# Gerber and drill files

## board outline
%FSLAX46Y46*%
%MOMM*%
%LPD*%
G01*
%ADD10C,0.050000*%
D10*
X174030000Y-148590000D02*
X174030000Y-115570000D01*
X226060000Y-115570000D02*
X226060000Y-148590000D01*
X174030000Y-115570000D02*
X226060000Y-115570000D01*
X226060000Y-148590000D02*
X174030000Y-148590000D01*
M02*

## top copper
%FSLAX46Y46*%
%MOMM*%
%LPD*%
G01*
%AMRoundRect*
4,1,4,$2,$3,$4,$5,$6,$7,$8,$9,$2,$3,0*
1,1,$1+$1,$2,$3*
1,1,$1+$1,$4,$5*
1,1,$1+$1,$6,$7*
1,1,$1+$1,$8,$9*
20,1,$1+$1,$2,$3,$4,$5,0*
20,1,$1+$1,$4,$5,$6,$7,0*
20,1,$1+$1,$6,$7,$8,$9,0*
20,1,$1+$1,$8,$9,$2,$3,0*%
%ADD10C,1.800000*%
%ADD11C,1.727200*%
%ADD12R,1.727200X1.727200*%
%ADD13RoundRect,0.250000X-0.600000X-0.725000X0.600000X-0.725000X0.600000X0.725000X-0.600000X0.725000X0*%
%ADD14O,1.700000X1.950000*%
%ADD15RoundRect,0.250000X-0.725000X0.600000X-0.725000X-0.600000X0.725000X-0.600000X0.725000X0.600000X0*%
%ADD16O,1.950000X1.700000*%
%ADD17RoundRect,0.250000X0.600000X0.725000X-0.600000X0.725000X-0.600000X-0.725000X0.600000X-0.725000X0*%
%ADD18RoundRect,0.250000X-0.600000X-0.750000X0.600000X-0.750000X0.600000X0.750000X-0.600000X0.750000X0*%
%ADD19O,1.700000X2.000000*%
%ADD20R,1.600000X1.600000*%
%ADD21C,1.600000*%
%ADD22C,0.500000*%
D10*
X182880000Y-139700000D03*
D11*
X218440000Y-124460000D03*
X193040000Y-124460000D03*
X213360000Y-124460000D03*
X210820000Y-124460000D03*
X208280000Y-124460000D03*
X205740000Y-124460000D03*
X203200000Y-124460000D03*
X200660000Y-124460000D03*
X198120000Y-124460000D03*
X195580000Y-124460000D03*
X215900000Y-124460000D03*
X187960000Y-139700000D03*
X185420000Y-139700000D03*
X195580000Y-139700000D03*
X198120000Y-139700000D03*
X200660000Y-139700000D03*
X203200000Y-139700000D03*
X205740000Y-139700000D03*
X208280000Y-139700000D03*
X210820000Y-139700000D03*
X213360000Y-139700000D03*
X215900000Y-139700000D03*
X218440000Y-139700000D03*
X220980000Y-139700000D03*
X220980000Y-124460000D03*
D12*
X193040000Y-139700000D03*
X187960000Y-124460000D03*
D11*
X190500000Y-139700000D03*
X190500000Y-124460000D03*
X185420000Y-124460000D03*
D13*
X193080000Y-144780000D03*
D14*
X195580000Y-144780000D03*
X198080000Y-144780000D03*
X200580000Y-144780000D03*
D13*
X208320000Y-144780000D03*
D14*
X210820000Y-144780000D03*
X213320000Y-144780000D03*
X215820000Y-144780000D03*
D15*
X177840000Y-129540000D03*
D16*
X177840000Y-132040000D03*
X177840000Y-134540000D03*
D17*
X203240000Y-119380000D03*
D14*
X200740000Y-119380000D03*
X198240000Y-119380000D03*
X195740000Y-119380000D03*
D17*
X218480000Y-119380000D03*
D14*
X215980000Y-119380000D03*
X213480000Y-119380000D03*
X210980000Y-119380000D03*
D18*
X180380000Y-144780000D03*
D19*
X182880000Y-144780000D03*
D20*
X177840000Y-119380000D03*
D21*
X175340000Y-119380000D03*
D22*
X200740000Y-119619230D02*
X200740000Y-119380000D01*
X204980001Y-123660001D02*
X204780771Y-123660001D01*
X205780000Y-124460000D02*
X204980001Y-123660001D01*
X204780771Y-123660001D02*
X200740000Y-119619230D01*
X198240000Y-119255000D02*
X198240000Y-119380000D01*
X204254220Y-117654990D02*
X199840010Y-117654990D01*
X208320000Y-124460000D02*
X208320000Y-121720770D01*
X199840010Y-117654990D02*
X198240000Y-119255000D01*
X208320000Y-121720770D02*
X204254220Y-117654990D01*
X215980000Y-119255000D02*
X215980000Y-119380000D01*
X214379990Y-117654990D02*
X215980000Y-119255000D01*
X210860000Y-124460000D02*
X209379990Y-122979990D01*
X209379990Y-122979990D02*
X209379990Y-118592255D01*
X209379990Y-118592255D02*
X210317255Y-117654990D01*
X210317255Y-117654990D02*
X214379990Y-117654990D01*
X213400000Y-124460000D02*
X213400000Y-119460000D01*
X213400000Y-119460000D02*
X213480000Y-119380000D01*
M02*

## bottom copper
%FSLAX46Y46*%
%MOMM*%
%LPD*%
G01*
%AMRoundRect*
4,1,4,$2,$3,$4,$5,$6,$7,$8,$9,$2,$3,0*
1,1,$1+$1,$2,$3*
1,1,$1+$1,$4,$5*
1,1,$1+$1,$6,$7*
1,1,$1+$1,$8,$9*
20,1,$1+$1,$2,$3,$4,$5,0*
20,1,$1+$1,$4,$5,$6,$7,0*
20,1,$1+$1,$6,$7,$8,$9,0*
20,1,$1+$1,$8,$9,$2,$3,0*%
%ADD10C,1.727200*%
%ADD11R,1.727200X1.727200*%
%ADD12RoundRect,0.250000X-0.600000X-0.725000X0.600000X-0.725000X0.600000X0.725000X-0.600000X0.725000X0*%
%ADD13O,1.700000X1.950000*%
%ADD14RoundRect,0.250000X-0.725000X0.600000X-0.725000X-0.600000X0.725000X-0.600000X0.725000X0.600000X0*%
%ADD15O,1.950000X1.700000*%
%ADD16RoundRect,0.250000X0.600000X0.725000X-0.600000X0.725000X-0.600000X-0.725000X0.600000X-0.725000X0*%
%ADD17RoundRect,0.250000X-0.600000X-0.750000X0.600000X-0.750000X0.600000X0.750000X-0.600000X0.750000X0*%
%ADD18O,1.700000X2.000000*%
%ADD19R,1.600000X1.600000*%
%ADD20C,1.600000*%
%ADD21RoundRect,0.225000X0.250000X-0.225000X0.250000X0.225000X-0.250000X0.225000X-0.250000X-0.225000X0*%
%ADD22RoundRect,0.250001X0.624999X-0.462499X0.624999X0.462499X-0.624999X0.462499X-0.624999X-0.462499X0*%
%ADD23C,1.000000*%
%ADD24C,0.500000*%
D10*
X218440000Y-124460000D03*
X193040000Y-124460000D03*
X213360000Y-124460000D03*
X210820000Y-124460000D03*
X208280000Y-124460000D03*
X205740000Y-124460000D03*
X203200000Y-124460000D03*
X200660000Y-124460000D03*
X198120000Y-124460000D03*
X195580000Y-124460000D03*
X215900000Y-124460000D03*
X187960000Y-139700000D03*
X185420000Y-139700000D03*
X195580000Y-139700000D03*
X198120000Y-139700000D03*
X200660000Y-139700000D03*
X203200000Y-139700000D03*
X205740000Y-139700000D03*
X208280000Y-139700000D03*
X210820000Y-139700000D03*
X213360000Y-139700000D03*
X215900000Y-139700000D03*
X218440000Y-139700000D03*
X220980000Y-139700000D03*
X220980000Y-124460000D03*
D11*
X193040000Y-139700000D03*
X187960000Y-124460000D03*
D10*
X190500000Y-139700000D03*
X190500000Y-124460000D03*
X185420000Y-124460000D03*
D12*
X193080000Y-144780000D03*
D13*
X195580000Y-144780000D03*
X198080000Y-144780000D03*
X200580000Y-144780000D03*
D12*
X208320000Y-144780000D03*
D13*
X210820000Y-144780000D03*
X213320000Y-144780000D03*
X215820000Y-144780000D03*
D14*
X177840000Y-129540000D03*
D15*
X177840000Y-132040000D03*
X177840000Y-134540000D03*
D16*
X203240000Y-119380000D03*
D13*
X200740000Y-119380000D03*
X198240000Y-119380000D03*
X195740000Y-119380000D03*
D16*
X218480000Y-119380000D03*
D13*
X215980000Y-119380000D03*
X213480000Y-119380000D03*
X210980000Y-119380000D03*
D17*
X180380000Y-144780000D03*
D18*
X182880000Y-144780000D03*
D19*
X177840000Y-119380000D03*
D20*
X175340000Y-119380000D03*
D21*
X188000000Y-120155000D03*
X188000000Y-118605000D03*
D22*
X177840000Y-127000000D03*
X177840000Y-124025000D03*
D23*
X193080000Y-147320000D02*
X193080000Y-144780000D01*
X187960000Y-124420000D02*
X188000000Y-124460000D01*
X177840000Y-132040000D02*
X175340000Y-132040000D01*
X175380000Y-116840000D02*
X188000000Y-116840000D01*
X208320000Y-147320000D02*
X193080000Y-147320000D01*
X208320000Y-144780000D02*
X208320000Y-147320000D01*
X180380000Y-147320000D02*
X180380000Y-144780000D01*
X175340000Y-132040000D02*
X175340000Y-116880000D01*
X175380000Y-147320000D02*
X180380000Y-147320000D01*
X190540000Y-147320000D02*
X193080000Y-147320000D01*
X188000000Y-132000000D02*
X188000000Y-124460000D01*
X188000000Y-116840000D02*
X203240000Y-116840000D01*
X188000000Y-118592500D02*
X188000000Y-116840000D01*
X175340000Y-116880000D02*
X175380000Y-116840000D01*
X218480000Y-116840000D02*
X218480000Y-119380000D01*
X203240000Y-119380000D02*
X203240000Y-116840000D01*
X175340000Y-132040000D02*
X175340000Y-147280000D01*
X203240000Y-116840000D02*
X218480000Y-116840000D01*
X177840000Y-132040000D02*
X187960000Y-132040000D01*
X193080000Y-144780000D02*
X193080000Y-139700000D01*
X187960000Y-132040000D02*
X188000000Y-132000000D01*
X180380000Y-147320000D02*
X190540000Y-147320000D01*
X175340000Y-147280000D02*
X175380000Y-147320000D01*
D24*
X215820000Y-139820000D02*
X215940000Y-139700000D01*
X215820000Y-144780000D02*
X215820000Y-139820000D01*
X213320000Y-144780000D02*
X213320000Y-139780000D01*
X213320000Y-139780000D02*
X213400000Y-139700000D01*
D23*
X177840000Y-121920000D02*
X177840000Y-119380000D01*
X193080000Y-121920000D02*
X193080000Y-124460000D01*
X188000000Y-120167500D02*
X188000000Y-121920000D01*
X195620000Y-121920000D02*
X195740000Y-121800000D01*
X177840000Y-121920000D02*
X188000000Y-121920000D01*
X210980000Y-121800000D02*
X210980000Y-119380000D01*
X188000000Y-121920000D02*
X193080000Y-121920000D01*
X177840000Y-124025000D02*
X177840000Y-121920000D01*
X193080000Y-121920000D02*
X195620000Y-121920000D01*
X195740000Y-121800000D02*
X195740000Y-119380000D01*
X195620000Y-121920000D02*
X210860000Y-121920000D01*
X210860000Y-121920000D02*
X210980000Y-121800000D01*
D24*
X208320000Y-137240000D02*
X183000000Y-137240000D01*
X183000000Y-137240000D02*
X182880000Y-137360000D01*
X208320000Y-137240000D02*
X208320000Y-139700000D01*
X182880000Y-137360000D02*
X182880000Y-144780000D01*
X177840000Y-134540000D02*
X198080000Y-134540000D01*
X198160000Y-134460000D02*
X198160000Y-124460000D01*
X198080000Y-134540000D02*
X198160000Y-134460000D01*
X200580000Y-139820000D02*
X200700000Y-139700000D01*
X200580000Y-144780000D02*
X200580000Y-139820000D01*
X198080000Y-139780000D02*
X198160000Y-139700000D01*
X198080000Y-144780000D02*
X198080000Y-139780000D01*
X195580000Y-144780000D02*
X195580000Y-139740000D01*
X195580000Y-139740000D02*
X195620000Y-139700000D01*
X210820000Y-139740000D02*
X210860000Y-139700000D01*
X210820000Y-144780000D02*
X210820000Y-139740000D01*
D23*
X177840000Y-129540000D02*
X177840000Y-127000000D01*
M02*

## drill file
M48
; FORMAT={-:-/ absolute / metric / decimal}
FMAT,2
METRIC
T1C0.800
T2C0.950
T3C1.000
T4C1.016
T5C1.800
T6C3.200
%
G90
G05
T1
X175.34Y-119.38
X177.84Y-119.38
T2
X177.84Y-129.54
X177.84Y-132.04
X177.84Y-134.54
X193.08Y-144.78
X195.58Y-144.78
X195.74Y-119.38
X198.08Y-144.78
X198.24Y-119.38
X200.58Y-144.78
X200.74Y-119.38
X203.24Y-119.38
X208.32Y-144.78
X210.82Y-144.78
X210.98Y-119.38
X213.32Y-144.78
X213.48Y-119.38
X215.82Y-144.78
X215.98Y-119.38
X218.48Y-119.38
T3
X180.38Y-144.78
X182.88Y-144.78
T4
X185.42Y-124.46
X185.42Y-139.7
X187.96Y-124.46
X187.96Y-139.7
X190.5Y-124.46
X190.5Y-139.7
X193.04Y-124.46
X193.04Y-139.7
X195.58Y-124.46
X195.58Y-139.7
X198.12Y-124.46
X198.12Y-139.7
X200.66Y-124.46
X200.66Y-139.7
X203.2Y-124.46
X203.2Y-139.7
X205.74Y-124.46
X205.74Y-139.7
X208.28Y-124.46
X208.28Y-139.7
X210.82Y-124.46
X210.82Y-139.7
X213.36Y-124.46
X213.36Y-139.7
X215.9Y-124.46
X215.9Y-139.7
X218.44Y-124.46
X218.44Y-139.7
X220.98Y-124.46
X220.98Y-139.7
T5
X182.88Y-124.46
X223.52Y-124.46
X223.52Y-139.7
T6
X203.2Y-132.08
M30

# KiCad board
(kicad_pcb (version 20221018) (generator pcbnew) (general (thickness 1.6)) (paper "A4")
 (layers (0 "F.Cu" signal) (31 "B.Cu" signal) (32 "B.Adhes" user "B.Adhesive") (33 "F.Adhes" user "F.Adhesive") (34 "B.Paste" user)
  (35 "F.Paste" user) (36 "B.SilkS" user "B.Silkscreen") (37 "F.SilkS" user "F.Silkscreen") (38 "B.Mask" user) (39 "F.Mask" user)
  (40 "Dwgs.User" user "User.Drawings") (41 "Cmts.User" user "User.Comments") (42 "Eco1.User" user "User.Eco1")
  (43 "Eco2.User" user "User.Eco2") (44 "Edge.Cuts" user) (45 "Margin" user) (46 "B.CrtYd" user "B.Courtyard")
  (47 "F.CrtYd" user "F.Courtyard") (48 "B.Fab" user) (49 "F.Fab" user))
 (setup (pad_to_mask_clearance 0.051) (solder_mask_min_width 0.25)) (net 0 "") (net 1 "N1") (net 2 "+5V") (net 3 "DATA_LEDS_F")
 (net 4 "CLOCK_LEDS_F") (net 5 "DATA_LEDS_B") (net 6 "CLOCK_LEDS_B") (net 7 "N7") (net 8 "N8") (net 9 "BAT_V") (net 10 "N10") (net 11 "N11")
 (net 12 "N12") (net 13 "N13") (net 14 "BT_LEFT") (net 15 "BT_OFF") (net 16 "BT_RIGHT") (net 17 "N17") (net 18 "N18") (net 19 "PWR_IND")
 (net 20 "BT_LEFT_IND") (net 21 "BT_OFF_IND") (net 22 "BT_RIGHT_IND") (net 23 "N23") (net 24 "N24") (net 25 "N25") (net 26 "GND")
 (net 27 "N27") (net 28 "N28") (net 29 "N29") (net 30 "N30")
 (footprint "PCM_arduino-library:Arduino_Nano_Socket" (layer "F.Cu") (at 224.79 132.08 90)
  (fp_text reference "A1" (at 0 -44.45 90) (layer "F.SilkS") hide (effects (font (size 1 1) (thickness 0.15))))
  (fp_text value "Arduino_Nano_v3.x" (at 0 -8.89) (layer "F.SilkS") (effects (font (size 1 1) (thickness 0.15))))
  (pad "" connect circle (at -7.62 -41.91 90) (size 1.8 1.8) (layers "F.Cu" "F.Mask"))
  (pad "" np_thru_hole circle (at -7.62 -1.27 90) (size 1.8 1.8) (drill 1.8) (layers "F&B.Cu" "*.Mask"))
  (pad "" np_thru_hole circle (at 7.62 -41.91 90) (size 1.8 1.8) (drill 1.8) (layers "F&B.Cu" "*.Mask"))
  (pad "" np_thru_hole circle (at 7.62 -1.27 90) (size 1.8 1.8) (drill 1.8) (layers "F&B.Cu" "*.Mask"))
  (pad "3V3" thru_hole circle (at 7.62 -6.35 90) (size 1.7272 1.7272) (drill 1.016) (layers "*.Cu" "*.Mask") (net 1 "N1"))
  (pad "5V" thru_hole circle (at 7.62 -31.75 90) (size 1.7272 1.7272) (drill 1.016) (layers "*.Cu" "*.Mask") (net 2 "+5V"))
  (pad "A0" thru_hole circle (at 7.62 -11.43 90) (size 1.7272 1.7272) (drill 1.016) (layers "*.Cu" "*.Mask") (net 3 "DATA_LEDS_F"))
  (pad "A1" thru_hole circle (at 7.62 -13.97 90) (size 1.7272 1.7272) (drill 1.016) (layers "*.Cu" "*.Mask") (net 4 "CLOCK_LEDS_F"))
  (pad "A2" thru_hole circle (at 7.62 -16.51 90) (size 1.7272 1.7272) (drill 1.016) (layers "*.Cu" "*.Mask") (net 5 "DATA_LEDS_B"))
  (pad "A3" thru_hole circle (at 7.62 -19.05 90) (size 1.7272 1.7272) (drill 1.016) (layers "*.Cu" "*.Mask") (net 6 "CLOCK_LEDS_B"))
  (pad "A4" thru_hole circle (at 7.62 -21.59 90) (size 1.7272 1.7272) (drill 1.016) (layers "*.Cu" "*.Mask") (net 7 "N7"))
  (pad "A5" thru_hole circle (at 7.62 -24.13 90) (size 1.7272 1.7272) (drill 1.016) (layers "*.Cu" "*.Mask") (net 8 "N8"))
  (pad "A6" thru_hole circle (at 7.62 -26.67 90) (size 1.7272 1.7272) (drill 1.016) (layers "*.Cu" "*.Mask") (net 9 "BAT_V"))
  (pad "A7" thru_hole circle (at 7.62 -29.21 90) (size 1.7272 1.7272) (drill 1.016) (layers "*.Cu" "*.Mask") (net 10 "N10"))
  (pad "AREF" thru_hole circle (at 7.62 -8.89 90) (size 1.7272 1.7272) (drill 1.016) (layers "*.Cu" "*.Mask") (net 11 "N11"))
  (pad "D0" thru_hole circle (at -7.62 -36.83 90) (size 1.7272 1.7272) (drill 1.016) (layers "*.Cu" "*.Mask") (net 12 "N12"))
  (pad "D1" thru_hole circle (at -7.62 -39.37 90) (size 1.7272 1.7272) (drill 1.016) (layers "*.Cu" "*.Mask") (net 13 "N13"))
  (pad "D2" thru_hole circle (at -7.62 -29.21 90) (size 1.7272 1.7272) (drill 1.016) (layers "*.Cu" "*.Mask") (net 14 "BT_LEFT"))
  (pad "D3" thru_hole circle (at -7.62 -26.67 90) (size 1.7272 1.7272) (drill 1.016) (layers "*.Cu" "*.Mask") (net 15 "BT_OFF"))
  (pad "D4" thru_hole circle (at -7.62 -24.13 90) (size 1.7272 1.7272) (drill 1.016) (layers "*.Cu" "*.Mask") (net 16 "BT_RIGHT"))
  (pad "D5" thru_hole circle (at -7.62 -21.59 90) (size 1.7272 1.7272) (drill 1.016) (layers "*.Cu" "*.Mask") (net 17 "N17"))
  (pad "D6" thru_hole circle (at -7.62 -19.05 90) (size 1.7272 1.7272) (drill 1.016) (layers "*.Cu" "*.Mask") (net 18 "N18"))
  (pad "D7" thru_hole circle (at -7.62 -16.51 90) (size 1.7272 1.7272) (drill 1.016) (layers "*.Cu" "*.Mask") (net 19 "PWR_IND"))
  (pad "D8" thru_hole circle (at -7.62 -13.97 90) (size 1.7272 1.7272) (drill 1.016) (layers "*.Cu" "*.Mask") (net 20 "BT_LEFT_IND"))
  (pad "D9" thru_hole circle (at -7.62 -11.43 90) (size 1.7272 1.7272) (drill 1.016) (layers "*.Cu" "*.Mask") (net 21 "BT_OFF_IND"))
  (pad "D10" thru_hole circle (at -7.62 -8.89 90) (size 1.7272 1.7272) (drill 1.016) (layers "*.Cu" "*.Mask") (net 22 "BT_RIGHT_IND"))
  (pad "D11" thru_hole circle (at -7.62 -6.35 90) (size 1.7272 1.7272) (drill 1.016) (layers "*.Cu" "*.Mask") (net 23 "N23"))
  (pad "D12" thru_hole circle (at -7.62 -3.81 90) (size 1.7272 1.7272) (drill 1.016) (layers "*.Cu" "*.Mask") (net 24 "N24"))
  (pad "D13" thru_hole circle (at 7.62 -3.81 90) (size 1.7272 1.7272) (drill 1.016) (layers "*.Cu" "*.Mask") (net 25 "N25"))
  (pad "GND1" thru_hole rect (at -7.62 -31.75 90) (size 1.7272 1.7272) (drill 1.016) (layers "*.Cu" "*.Mask") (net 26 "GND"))
  (pad "GND2" thru_hole rect (at 7.62 -36.83 90) (size 1.7272 1.7272) (drill 1.016) (layers "*.Cu" "*.Mask") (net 26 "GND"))
  (pad "RST1" thru_hole circle (at -7.62 -34.29 90) (size 1.7272 1.7272) (drill 1.016) (layers "*.Cu" "*.Mask") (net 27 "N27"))
  (pad "RST2" thru_hole circle (at 7.62 -34.29 90) (size 1.7272 1.7272) (drill 1.016) (layers "*.Cu" "*.Mask") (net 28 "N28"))
  (pad "VIN" thru_hole circle (at 7.62 -39.37 90) (size 1.7272 1.7272) (drill 1.016) (layers "*.Cu" "*.Mask") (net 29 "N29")))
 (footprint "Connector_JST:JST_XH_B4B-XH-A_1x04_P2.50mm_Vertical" (layer "F.Cu") (at 193.08 144.78)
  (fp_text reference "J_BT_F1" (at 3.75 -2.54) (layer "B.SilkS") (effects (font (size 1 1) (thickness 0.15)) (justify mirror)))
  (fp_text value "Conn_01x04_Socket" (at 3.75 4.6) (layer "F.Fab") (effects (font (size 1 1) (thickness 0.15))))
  (pad "1" thru_hole roundrect (at 0 0) (size 1.7 1.95) (drill 0.95) (layers "*.Cu" "*.Mask") (roundrect_rratio 0.147059) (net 26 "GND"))
  (pad "2" thru_hole oval (at 2.5 0) (size 1.7 1.95) (drill 0.95) (layers "*.Cu" "*.Mask") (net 14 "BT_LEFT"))
  (pad "3" thru_hole oval (at 5 0) (size 1.7 1.95) (drill 0.95) (layers "*.Cu" "*.Mask") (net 15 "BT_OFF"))
  (pad "4" thru_hole oval (at 7.5 0) (size 1.7 1.95) (drill 0.95) (layers "*.Cu" "*.Mask") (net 16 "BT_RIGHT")))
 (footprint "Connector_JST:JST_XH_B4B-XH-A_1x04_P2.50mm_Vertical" (layer "F.Cu") (at 208.32 144.78)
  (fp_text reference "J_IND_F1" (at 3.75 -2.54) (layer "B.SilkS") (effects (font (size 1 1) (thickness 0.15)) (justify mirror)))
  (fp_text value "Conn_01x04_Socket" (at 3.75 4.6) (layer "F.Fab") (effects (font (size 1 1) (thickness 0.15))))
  (pad "1" thru_hole roundrect (at 0 0) (size 1.7 1.95) (drill 0.95) (layers "*.Cu" "*.Mask") (roundrect_rratio 0.147059) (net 26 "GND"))
  (pad "2" thru_hole oval (at 2.5 0) (size 1.7 1.95) (drill 0.95) (layers "*.Cu" "*.Mask") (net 20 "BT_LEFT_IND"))
  (pad "3" thru_hole oval (at 5 0) (size 1.7 1.95) (drill 0.95) (layers "*.Cu" "*.Mask") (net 21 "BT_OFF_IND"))
  (pad "4" thru_hole oval (at 7.5 0) (size 1.7 1.95) (drill 0.95) (layers "*.Cu" "*.Mask") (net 22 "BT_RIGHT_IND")))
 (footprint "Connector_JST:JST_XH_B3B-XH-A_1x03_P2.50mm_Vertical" (layer "F.Cu") (at 177.84 129.54 -90)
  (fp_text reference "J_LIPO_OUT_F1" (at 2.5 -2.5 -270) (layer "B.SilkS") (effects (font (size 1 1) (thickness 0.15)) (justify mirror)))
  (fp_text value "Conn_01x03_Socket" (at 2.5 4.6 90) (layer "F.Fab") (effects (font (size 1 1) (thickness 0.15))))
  (pad "1" thru_hole roundrect (at 0 0 270) (size 1.7 1.95) (drill 0.95) (layers "*.Cu" "*.Mask") (roundrect_rratio 0.147059) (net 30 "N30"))
  (pad "2" thru_hole oval (at 2.5 0 270) (size 1.7 1.95) (drill 0.95) (layers "*.Cu" "*.Mask") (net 26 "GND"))
  (pad "3" thru_hole oval (at 5 0 270) (size 1.7 1.95) (drill 0.95) (layers "*.Cu" "*.Mask") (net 9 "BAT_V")))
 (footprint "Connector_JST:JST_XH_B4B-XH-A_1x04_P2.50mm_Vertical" (layer "F.Cu") (at 203.24 119.38 180)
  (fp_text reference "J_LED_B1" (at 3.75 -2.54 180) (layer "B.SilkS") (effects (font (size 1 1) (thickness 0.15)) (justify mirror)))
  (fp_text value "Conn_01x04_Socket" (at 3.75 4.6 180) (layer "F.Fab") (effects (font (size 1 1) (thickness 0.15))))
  (pad "1" thru_hole roundrect (at 0 0 180) (size 1.7 1.95) (drill 0.95) (layers "*.Cu" "*.Mask") (roundrect_rratio 0.147059) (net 26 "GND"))
  (pad "2" thru_hole oval (at 2.5 0 180) (size 1.7 1.95) (drill 0.95) (layers "*.Cu" "*.Mask") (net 6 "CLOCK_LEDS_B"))
  (pad "3" thru_hole oval (at 5 0 180) (size 1.7 1.95) (drill 0.95) (layers "*.Cu" "*.Mask") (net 5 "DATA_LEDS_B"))
  (pad "4" thru_hole oval (at 7.5 0 180) (size 1.7 1.95) (drill 0.95) (layers "*.Cu" "*.Mask") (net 2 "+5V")))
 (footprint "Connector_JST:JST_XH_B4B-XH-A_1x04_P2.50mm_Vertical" (layer "F.Cu") (at 218.48 119.38 180)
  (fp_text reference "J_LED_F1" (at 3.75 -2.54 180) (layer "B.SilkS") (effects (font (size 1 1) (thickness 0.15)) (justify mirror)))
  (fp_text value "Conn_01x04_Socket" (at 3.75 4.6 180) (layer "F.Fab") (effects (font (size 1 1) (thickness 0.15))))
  (pad "1" thru_hole roundrect (at 0 0 180) (size 1.7 1.95) (drill 0.95) (layers "*.Cu" "*.Mask") (roundrect_rratio 0.147059) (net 26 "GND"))
  (pad "2" thru_hole oval (at 2.5 0 180) (size 1.7 1.95) (drill 0.95) (layers "*.Cu" "*.Mask") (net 4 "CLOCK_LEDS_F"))
  (pad "3" thru_hole oval (at 5 0 180) (size 1.7 1.95) (drill 0.95) (layers "*.Cu" "*.Mask") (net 3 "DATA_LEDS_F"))
  (pad "4" thru_hole oval (at 7.5 0 180) (size 1.7 1.95) (drill 0.95) (layers "*.Cu" "*.Mask") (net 2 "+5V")))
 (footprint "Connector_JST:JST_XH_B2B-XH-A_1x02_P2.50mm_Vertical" (layer "F.Cu") (at 180.38 144.78)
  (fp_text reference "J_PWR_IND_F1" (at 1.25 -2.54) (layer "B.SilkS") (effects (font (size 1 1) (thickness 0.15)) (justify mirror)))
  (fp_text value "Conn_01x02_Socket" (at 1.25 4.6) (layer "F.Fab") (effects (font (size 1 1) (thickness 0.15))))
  (pad "1" thru_hole roundrect (at 0 0) (size 1.7 2) (drill 1) (layers "*.Cu" "*.Mask") (roundrect_rratio 0.147059) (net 26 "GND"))
  (pad "2" thru_hole oval (at 2.5 0) (size 1.7 2) (drill 1) (layers "*.Cu" "*.Mask") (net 19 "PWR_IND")))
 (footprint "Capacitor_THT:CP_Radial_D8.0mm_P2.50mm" (layer "F.Cu") (at 177.84 119.38 180)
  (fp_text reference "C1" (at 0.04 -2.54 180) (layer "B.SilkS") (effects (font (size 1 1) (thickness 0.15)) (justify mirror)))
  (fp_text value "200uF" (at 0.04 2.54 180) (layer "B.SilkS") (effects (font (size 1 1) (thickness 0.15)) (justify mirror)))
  (pad "1" thru_hole rect (at 0 0 180) (size 1.6 1.6) (drill 0.8) (layers "*.Cu" "*.Mask") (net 2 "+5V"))
  (pad "2" thru_hole circle (at 2.5 0 180) (size 1.6 1.6) (drill 0.8) (layers "*.Cu" "*.Mask") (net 26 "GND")))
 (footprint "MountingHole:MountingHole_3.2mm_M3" (layer "F.Cu") (at 203.2 132.08)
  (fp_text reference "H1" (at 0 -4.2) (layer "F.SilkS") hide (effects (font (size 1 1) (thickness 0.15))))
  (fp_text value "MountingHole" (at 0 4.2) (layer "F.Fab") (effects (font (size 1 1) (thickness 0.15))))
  (pad "" np_thru_hole circle (at 0 0) (size 3.2 3.2) (drill 3.2) (layers "*.Cu" "*.Mask")))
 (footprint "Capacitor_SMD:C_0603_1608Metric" (layer "B.Cu") (at 188 119.38 90)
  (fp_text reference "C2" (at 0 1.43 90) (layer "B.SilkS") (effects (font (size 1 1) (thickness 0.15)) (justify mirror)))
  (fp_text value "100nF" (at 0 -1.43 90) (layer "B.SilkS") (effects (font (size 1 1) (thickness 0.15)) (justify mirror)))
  (pad "1" smd roundrect (at -0.775 0 90) (size 0.9 0.95) (layers "B.Cu" "B.Paste" "B.Mask") (roundrect_rratio 0.25) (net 2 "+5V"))
  (pad "2" smd roundrect (at 0.775 0 90) (size 0.9 0.95) (layers "B.Cu" "B.Paste" "B.Mask") (roundrect_rratio 0.25) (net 26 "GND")))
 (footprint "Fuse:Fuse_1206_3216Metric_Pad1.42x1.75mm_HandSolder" (layer "B.Cu") (at 177.84 125.5125 90)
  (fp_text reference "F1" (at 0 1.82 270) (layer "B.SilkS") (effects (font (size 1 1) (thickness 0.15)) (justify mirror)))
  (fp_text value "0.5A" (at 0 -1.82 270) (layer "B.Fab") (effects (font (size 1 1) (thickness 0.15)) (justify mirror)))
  (pad "1" smd roundrect (at -1.4875 0 90) (size 1.425 1.75) (layers "B.Cu" "B.Paste" "B.Mask") (roundrect_rratio 0.175439) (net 30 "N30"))
  (pad "2" smd roundrect (at 1.4875 0 90) (size 1.425 1.75) (layers "B.Cu" "B.Paste" "B.Mask") (roundrect_rratio 0.175439) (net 2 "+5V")))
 (gr_line (start 174.03 148.59) (end 174.03 115.57) (stroke (width 0.05) (type solid)) (layer "Edge.Cuts"))
 (gr_line (start 226.06 115.57) (end 226.06 148.59) (stroke (width 0.05) (type solid)) (layer "Edge.Cuts"))
 (gr_line (start 174.03 115.57) (end 226.06 115.57) (stroke (width 0.05) (type solid)) (layer "Edge.Cuts"))
 (gr_line (start 226.06 148.59) (end 174.03 148.59) (stroke (width 0.05) (type solid)) (layer "Edge.Cuts"))
 (segment (start 193.08 147.32) (end 193.08 144.78) (width 1) (layer "B.Cu") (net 26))
 (segment (start 187.96 124.42) (end 188 124.46) (width 1) (layer "B.Cu") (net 26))
 (segment (start 177.84 132.04) (end 175.34 132.04) (width 1) (layer "B.Cu") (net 26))
 (segment (start 175.38 116.84) (end 188 116.84) (width 1) (layer "B.Cu") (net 26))
 (segment (start 208.32 147.32) (end 193.08 147.32) (width 1) (layer "B.Cu") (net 26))
 (segment (start 208.32 144.78) (end 208.32 147.32) (width 1) (layer "B.Cu") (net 26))
 (segment (start 180.38 147.32) (end 180.38 144.78) (width 1) (layer "B.Cu") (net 26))
 (segment (start 175.34 132.04) (end 175.34 116.88) (width 1) (layer "B.Cu") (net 26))
 (segment (start 175.38 147.32) (end 180.38 147.32) (width 1) (layer "B.Cu") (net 26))
 (segment (start 190.54 147.32) (end 193.08 147.32) (width 1) (layer "B.Cu") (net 26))
 (segment (start 188 132) (end 188 124.46) (width 1) (layer "B.Cu") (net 26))
 (segment (start 188 116.84) (end 203.24 116.84) (width 1) (layer "B.Cu") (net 26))
 (segment (start 188 118.5925) (end 188 116.84) (width 1) (layer "B.Cu") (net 26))
 (segment (start 175.34 116.88) (end 175.38 116.84) (width 1) (layer "B.Cu") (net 26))
 (segment (start 218.48 116.84) (end 218.48 119.38) (width 1) (layer "B.Cu") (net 26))
 (segment (start 203.24 119.38) (end 203.24 116.84) (width 1) (layer "B.Cu") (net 26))
 (segment (start 175.34 132.04) (end 175.34 147.28) (width 1) (layer "B.Cu") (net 26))
 (segment (start 203.24 116.84) (end 218.48 116.84) (width 1) (layer "B.Cu") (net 26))
 (segment (start 177.84 132.04) (end 187.96 132.04) (width 1) (layer "B.Cu") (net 26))
 (segment (start 193.08 144.78) (end 193.08 139.7) (width 1) (layer "B.Cu") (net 26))
 (segment (start 187.96 132.04) (end 188 132) (width 1) (layer "B.Cu") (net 26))
 (segment (start 180.38 147.32) (end 190.54 147.32) (width 1) (layer "B.Cu") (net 26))
 (segment (start 175.34 147.28) (end 175.38 147.32) (width 1) (layer "B.Cu") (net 26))
 (segment (start 215.82 139.82) (end 215.94 139.7) (width 0.5) (layer "B.Cu") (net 22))
 (segment (start 215.82 144.78) (end 215.82 139.82) (width 0.5) (layer "B.Cu") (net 22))
 (segment (start 213.32 144.78) (end 213.32 139.78) (width 0.5) (layer "B.Cu") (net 21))
 (segment (start 213.32 139.78) (end 213.4 139.7) (width 0.5) (layer "B.Cu") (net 21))
 (segment (start 177.84 121.92) (end 177.84 119.38) (width 1) (layer "B.Cu") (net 2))
 (segment (start 193.08 121.92) (end 193.08 124.46) (width 1) (layer "B.Cu") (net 2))
 (segment (start 188 120.1675) (end 188 121.92) (width 1) (layer "B.Cu") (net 2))
 (segment (start 195.62 121.92) (end 195.74 121.8) (width 1) (layer "B.Cu") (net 2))
 (segment (start 177.84 121.92) (end 188 121.92) (width 1) (layer "B.Cu") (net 2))
 (segment (start 210.98 121.8) (end 210.98 119.38) (width 1) (layer "B.Cu") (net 2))
 (segment (start 188 121.92) (end 193.08 121.92) (width 1) (layer "B.Cu") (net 2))
 (segment (start 177.84 124.025) (end 177.84 121.92) (width 1) (layer "B.Cu") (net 2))
 (segment (start 193.08 121.92) (end 195.62 121.92) (width 1) (layer "B.Cu") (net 2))
 (segment (start 195.74 121.8) (end 195.74 119.38) (width 1) (layer "B.Cu") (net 2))
 (segment (start 195.62 121.92) (end 210.86 121.92) (width 1) (layer "B.Cu") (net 2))
 (segment (start 210.86 121.92) (end 210.98 121.8) (width 1) (layer "B.Cu") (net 2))
 (segment (start 208.32 137.24) (end 183 137.24) (width 0.5) (layer "B.Cu") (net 19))
 (segment (start 183 137.24) (end 182.88 137.36) (width 0.5) (layer "B.Cu") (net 19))
 (segment (start 208.32 137.24) (end 208.32 139.7) (width 0.5) (layer "B.Cu") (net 19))
 (segment (start 182.88 137.36) (end 182.88 144.78) (width 0.5) (layer "B.Cu") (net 19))
 (segment (start 177.84 134.54) (end 198.08 134.54) (width 0.5) (layer "B.Cu") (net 9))
 (segment (start 198.16 134.46) (end 198.16 124.46) (width 0.5) (layer "B.Cu") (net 9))
 (segment (start 198.08 134.54) (end 198.16 134.46) (width 0.5) (layer "B.Cu") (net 9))
 (segment (start 200.58 139.82) (end 200.7 139.7) (width 0.5) (layer "B.Cu") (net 16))
 (segment (start 200.58 144.78) (end 200.58 139.82) (width 0.5) (layer "B.Cu") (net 16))
 (segment (start 198.08 139.78) (end 198.16 139.7) (width 0.5) (layer "B.Cu") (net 15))
 (segment (start 198.08 144.78) (end 198.08 139.78) (width 0.5) (layer "B.Cu") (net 15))
 (segment (start 200.74 119.61923) (end 200.74 119.38) (width 0.5) (layer "F.Cu") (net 6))
 (segment (start 204.980001 123.660001) (end 204.780771 123.660001) (width 0.5) (layer "F.Cu") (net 6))
 (segment (start 205.78 124.46) (end 204.980001 123.660001) (width 0.5) (layer "F.Cu") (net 6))
 (segment (start 204.780771 123.660001) (end 200.74 119.61923) (width 0.5) (layer "F.Cu") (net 6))
 (segment (start 198.24 119.255) (end 198.24 119.38) (width 0.5) (layer "F.Cu") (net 5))
 (segment (start 204.25422 117.65499) (end 199.84001 117.65499) (width 0.5) (layer "F.Cu") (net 5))
 (segment (start 208.32 124.46) (end 208.32 121.72077) (width 0.5) (layer "F.Cu") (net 5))
 (segment (start 199.84001 117.65499) (end 198.24 119.255) (width 0.5) (layer "F.Cu") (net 5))
 (segment (start 208.32 121.72077) (end 204.25422 117.65499) (width 0.5) (layer "F.Cu") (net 5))
 (segment (start 215.98 119.255) (end 215.98 119.38) (width 0.5) (layer "F.Cu") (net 4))
 (segment (start 214.37999 117.65499) (end 215.98 119.255) (width 0.5) (layer "F.Cu") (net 4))
 (segment (start 210.86 124.46) (end 209.37999 122.97999) (width 0.5) (layer "F.Cu") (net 4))
 (segment (start 209.37999 122.97999) (end 209.37999 118.592255) (width 0.5) (layer "F.Cu") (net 4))
 (segment (start 209.37999 118.592255) (end 210.317255 117.65499) (width 0.5) (layer "F.Cu") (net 4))
 (segment (start 210.317255 117.65499) (end 214.37999 117.65499) (width 0.5) (layer "F.Cu") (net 4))
 (segment (start 213.4 124.46) (end 213.4 119.46) (width 0.5) (layer "F.Cu") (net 3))
 (segment (start 213.4 119.46) (end 213.48 119.38) (width 0.5) (layer "F.Cu") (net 3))
 (segment (start 195.58 144.78) (end 195.58 139.74) (width 0.5) (layer "B.Cu") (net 14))
 (segment (start 195.58 139.74) (end 195.62 139.7) (width 0.5) (layer "B.Cu") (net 14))
 (segment (start 210.82 139.74) (end 210.86 139.7) (width 0.5) (layer "B.Cu") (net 20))
 (segment (start 210.82 144.78) (end 210.82 139.74) (width 0.5) (layer "B.Cu") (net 20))
 (segment (start 177.84 129.54) (end 177.84 127) (width 1) (layer "B.Cu") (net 30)))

